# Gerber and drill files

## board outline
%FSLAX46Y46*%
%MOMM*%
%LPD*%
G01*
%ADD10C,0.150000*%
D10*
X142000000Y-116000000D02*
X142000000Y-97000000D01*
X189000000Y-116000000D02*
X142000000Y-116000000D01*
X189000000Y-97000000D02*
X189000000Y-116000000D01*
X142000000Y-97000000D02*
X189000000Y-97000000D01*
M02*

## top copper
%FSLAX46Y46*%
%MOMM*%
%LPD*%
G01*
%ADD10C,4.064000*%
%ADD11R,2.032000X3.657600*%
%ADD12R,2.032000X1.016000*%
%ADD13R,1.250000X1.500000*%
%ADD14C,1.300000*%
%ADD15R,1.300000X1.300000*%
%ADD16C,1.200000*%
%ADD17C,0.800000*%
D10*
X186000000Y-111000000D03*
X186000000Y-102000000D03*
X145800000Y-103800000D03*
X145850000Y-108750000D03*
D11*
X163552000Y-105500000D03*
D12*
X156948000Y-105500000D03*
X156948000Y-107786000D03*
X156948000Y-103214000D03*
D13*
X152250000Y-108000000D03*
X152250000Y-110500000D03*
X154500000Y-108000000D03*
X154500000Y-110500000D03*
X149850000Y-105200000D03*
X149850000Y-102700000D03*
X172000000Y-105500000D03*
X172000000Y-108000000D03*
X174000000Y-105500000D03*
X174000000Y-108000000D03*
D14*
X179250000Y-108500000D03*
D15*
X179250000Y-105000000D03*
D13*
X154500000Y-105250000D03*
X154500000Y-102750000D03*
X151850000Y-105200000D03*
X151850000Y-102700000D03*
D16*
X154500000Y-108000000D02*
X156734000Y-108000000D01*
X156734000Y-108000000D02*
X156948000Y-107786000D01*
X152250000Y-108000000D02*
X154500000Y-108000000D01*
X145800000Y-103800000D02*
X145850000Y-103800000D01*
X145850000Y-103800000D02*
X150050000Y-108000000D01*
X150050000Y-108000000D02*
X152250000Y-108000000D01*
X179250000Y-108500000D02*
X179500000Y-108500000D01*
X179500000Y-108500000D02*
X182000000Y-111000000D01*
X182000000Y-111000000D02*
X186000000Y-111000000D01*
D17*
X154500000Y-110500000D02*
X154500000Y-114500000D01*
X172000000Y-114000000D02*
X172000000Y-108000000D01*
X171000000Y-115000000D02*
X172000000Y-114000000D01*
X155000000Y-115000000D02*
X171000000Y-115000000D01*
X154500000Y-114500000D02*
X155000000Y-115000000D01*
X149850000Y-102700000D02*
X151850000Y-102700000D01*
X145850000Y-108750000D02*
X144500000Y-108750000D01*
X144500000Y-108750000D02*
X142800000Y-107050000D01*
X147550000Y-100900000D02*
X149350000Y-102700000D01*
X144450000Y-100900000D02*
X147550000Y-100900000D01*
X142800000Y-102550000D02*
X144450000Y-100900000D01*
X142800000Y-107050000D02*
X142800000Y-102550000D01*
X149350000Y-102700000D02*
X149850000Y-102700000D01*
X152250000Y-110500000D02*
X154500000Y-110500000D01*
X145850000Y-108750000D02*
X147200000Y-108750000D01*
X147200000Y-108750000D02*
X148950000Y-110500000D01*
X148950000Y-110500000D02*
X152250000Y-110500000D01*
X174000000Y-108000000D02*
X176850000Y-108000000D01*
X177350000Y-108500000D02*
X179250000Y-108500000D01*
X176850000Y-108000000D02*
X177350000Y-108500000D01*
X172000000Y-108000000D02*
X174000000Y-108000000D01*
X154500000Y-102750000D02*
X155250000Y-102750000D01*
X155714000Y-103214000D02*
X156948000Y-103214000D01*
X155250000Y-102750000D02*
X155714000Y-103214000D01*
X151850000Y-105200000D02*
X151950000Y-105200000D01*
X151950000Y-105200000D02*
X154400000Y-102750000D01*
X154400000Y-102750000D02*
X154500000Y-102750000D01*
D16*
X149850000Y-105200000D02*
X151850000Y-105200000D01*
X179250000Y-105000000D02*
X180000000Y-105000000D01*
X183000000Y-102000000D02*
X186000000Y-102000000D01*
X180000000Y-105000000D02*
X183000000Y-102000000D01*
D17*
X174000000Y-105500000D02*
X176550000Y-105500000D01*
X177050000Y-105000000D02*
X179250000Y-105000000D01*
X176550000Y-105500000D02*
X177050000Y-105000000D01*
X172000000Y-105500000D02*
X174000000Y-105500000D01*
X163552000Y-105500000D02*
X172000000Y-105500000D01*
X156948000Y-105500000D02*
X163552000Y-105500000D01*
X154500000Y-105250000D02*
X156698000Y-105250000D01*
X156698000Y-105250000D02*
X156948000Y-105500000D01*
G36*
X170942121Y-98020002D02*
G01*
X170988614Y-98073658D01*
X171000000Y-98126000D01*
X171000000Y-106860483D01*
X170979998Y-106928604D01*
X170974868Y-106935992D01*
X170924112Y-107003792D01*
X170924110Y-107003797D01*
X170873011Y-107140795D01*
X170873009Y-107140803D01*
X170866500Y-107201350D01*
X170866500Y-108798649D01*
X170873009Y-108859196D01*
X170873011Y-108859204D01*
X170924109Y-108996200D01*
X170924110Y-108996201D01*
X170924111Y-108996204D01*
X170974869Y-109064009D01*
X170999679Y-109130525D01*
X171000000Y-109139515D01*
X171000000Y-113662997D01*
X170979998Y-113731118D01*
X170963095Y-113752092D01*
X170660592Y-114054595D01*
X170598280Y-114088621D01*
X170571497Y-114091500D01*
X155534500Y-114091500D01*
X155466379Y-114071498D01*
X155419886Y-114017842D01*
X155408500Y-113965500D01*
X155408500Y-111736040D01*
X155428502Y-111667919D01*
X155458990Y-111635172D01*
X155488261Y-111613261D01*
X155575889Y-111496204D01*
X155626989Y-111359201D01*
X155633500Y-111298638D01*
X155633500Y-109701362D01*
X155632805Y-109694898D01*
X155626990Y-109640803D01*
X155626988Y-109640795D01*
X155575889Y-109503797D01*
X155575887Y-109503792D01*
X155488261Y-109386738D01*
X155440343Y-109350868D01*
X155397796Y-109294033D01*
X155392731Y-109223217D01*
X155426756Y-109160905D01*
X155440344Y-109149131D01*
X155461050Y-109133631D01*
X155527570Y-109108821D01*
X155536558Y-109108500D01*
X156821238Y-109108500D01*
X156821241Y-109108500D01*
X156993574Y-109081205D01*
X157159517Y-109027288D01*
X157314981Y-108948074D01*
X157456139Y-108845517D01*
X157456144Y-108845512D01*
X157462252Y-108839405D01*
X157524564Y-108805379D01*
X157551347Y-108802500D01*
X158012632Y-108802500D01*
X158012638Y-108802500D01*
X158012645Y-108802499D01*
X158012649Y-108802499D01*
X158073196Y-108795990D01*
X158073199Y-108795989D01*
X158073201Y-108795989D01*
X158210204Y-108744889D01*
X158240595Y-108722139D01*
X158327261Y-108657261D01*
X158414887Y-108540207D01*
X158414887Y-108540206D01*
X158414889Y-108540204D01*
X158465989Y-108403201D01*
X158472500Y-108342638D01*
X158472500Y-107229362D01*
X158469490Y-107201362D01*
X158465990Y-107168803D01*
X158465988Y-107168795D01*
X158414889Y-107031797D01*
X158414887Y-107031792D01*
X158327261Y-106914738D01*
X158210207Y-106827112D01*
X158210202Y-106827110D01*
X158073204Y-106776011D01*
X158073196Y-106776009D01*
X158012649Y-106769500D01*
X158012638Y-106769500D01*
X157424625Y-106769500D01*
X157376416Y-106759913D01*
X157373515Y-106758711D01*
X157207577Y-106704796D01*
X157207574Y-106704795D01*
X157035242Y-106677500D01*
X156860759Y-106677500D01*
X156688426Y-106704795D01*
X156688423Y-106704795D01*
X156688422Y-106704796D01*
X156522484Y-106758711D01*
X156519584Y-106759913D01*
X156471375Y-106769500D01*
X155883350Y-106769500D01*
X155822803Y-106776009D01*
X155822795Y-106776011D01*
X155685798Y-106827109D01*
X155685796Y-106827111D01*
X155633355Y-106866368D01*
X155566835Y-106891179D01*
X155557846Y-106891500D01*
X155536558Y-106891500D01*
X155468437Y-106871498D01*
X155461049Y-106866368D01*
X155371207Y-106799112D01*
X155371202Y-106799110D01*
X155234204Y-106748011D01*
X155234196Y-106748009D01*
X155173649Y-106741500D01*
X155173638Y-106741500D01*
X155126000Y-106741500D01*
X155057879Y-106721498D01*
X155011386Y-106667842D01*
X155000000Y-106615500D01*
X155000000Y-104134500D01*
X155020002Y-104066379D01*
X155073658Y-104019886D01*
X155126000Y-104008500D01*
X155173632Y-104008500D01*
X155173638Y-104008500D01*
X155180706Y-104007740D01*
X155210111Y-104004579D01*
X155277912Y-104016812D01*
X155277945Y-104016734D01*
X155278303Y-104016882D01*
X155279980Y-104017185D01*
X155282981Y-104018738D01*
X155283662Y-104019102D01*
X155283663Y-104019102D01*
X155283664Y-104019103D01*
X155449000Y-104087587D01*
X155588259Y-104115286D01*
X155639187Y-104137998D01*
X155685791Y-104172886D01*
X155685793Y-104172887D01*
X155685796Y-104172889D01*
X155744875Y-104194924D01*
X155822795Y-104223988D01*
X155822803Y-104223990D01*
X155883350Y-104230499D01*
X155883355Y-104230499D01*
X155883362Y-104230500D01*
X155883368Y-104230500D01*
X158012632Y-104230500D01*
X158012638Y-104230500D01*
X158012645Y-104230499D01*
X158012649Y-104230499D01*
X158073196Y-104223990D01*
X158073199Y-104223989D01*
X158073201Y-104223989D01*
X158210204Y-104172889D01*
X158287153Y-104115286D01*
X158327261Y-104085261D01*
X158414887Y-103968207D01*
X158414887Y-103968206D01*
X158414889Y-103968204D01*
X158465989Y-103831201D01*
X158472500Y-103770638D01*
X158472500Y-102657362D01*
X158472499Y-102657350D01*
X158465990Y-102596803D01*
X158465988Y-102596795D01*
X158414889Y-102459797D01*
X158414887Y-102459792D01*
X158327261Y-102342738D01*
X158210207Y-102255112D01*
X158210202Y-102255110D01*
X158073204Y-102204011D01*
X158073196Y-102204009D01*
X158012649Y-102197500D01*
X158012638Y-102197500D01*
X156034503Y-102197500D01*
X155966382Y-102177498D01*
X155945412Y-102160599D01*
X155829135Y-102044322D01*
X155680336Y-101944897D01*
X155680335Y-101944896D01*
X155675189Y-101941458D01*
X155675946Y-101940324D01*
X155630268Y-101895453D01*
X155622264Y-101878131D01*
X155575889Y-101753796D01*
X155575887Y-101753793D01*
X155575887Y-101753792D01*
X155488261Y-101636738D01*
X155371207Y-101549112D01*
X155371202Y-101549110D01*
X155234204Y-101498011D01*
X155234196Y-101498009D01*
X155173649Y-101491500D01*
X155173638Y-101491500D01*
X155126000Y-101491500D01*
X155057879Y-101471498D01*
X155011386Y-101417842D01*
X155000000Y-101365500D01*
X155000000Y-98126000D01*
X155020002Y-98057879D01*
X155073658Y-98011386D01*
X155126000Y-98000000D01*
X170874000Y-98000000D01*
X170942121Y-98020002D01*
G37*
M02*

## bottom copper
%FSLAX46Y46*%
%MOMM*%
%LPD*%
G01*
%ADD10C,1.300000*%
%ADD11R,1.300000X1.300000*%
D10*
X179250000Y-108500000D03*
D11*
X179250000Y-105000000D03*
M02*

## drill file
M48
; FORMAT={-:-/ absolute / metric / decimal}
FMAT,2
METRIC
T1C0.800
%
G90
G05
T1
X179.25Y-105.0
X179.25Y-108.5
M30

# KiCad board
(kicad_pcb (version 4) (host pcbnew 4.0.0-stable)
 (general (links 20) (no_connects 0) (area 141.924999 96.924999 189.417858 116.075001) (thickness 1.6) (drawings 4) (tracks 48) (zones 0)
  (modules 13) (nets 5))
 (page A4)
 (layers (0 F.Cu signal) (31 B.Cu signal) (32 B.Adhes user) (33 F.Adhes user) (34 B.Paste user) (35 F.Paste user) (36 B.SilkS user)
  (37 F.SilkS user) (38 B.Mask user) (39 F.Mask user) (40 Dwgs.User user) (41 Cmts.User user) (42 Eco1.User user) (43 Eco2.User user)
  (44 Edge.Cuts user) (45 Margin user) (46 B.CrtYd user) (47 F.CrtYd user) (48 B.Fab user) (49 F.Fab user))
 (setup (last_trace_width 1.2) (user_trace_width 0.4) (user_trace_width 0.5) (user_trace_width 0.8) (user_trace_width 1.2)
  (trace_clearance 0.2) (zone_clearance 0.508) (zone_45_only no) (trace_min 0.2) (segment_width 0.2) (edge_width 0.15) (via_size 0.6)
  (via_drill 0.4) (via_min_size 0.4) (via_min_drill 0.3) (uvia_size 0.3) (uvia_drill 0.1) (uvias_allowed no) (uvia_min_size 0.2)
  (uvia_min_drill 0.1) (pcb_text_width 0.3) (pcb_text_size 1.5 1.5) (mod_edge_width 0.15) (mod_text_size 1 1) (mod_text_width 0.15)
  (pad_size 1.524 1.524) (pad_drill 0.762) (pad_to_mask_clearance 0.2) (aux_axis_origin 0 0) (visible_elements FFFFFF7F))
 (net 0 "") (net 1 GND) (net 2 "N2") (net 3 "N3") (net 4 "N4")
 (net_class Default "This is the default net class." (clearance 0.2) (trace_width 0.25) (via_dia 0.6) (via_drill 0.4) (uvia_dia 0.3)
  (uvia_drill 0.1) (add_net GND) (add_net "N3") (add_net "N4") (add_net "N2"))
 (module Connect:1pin (layer F.Cu) (at 186 111)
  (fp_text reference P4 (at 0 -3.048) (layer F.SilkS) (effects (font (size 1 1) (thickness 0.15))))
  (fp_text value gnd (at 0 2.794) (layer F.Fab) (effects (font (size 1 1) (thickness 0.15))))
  (pad 1 smd circle (at 0 0) (size 4.064 4.064) (layers F.Cu F.Paste F.Mask) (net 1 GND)))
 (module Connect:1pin (layer F.Cu) (at 186 102)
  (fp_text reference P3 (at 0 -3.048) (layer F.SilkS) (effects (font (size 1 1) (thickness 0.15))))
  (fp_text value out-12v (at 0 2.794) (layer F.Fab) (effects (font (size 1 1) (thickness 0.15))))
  (pad 1 smd circle (at 0 0) (size 4.064 4.064) (layers F.Cu F.Paste F.Mask) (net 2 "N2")))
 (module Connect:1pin (layer F.Cu) (at 145.8 103.8)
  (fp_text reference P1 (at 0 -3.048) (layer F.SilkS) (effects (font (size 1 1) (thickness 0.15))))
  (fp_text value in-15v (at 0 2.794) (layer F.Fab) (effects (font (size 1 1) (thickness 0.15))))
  (pad 1 smd circle (at 0 0) (size 4.064 4.064) (layers F.Cu F.Paste F.Mask) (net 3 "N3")))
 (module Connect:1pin (layer F.Cu) (at 145.85 108.75)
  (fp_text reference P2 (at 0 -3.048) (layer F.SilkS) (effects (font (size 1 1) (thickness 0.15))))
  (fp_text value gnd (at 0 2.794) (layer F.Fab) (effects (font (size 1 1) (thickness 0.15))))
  (pad 1 smd circle (at 0 0) (size 4.064 4.064) (layers F.Cu F.Paste F.Mask) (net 1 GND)))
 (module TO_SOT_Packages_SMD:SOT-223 (layer F.Cu) (at 160.25 105.5 270)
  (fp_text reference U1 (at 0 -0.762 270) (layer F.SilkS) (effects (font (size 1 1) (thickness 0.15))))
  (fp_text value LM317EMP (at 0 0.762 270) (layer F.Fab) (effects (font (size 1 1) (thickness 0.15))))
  (pad 2 smd rect (at 0 -3.302 270) (size 3.6576 2.032) (layers F.Cu F.Paste F.Mask) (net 2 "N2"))
  (pad 2 smd rect (at 0 3.302 270) (size 1.016 2.032) (layers F.Cu F.Paste F.Mask) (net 2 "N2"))
  (pad 3 smd rect (at 2.286 3.302 270) (size 1.016 2.032) (layers F.Cu F.Paste F.Mask) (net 3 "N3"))
  (pad 1 smd rect (at -2.286 3.302 270) (size 1.016 2.032) (layers F.Cu F.Paste F.Mask) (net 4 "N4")))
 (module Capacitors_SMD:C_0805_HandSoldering (layer F.Cu) (at 152.25 109.25 270)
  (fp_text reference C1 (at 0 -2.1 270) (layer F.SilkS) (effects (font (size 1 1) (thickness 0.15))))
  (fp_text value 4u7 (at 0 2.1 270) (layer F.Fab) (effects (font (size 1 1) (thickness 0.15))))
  (pad 1 smd rect (at -1.25 0 270) (size 1.5 1.25) (layers F.Cu F.Paste F.Mask) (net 3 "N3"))
  (pad 2 smd rect (at 1.25 0 270) (size 1.5 1.25) (layers F.Cu F.Paste F.Mask) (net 1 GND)))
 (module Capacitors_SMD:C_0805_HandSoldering (layer F.Cu) (at 154.5 109.25 270)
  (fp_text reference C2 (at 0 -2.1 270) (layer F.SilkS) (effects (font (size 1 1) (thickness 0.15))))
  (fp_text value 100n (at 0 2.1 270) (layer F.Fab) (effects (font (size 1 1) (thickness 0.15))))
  (pad 1 smd rect (at -1.25 0 270) (size 1.5 1.25) (layers F.Cu F.Paste F.Mask) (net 3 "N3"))
  (pad 2 smd rect (at 1.25 0 270) (size 1.5 1.25) (layers F.Cu F.Paste F.Mask) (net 1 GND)))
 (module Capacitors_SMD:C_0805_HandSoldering (layer F.Cu) (at 149.85 103.95 90)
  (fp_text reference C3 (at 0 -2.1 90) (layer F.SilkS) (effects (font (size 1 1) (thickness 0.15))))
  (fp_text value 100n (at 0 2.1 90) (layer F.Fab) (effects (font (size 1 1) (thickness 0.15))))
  (pad 1 smd rect (at -1.25 0 90) (size 1.5 1.25) (layers F.Cu F.Paste F.Mask) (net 4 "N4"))
  (pad 2 smd rect (at 1.25 0 90) (size 1.5 1.25) (layers F.Cu F.Paste F.Mask) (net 1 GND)))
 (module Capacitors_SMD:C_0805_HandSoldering (layer F.Cu) (at 172 106.75 270)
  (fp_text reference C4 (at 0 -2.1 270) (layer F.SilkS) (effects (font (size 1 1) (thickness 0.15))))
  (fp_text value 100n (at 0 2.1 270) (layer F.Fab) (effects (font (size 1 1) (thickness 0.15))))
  (pad 1 smd rect (at -1.25 0 270) (size 1.5 1.25) (layers F.Cu F.Paste F.Mask) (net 2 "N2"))
  (pad 2 smd rect (at 1.25 0 270) (size 1.5 1.25) (layers F.Cu F.Paste F.Mask) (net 1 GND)))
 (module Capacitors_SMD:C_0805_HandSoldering (layer F.Cu) (at 174 106.75 270)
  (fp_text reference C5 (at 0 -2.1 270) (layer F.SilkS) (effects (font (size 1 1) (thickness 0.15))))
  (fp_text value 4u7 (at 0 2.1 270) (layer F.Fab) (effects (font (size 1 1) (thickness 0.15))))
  (pad 1 smd rect (at -1.25 0 270) (size 1.5 1.25) (layers F.Cu F.Paste F.Mask) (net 2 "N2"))
  (pad 2 smd rect (at 1.25 0 270) (size 1.5 1.25) (layers F.Cu F.Paste F.Mask) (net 1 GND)))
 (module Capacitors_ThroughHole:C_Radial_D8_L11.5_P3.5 (layer F.Cu) (at 179.25 105 270)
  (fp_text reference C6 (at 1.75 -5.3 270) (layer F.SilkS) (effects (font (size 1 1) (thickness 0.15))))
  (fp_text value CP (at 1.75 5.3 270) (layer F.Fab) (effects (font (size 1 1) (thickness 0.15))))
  (pad 2 thru_hole circle (at 3.5 0 270) (size 1.3 1.3) (drill 0.8) (layers *.Cu *.Mask F.SilkS) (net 1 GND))
  (pad 1 thru_hole rect (at 0 0 270) (size 1.3 1.3) (drill 0.8) (layers *.Cu *.Mask F.SilkS) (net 2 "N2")))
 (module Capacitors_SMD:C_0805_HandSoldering (layer F.Cu) (at 154.5 104 90)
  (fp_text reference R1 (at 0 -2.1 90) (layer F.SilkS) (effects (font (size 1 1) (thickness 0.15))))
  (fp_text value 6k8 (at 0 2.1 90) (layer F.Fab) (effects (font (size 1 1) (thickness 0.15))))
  (pad 1 smd rect (at -1.25 0 90) (size 1.5 1.25) (layers F.Cu F.Paste F.Mask) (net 2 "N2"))
  (pad 2 smd rect (at 1.25 0 90) (size 1.5 1.25) (layers F.Cu F.Paste F.Mask) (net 4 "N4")))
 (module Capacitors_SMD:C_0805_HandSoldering (layer F.Cu) (at 151.85 103.95 90)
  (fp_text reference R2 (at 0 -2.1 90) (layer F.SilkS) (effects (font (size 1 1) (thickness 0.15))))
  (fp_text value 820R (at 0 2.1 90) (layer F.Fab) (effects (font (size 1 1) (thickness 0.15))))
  (pad 1 smd rect (at -1.25 0 90) (size 1.5 1.25) (layers F.Cu F.Paste F.Mask) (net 4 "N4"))
  (pad 2 smd rect (at 1.25 0 90) (size 1.5 1.25) (layers F.Cu F.Paste F.Mask) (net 1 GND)))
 (gr_line (start 142 116) (end 142 97) (angle 90) (layer Edge.Cuts) (width 0.15))
 (gr_line (start 189 116) (end 142 116) (angle 90) (layer Edge.Cuts) (width 0.15))
 (gr_line (start 189 97) (end 189 116) (angle 90) (layer Edge.Cuts) (width 0.15))
 (gr_line (start 142 97) (end 189 97) (angle 90) (layer Edge.Cuts) (width 0.15))
 (segment (start 154.5 108) (end 156.734 108) (width 1.2) (layer F.Cu) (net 3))
 (segment (start 156.734 108) (end 156.948 107.786) (width 1.2) (layer F.Cu) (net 3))
 (segment (start 152.25 108) (end 154.5 108) (width 1.2) (layer F.Cu) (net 3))
 (segment (start 145.8 103.8) (end 145.85 103.8) (width 1.2) (layer F.Cu) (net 3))
 (segment (start 145.85 103.8) (end 150.05 108) (width 1.2) (layer F.Cu) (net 3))
 (segment (start 150.05 108) (end 152.25 108) (width 1.2) (layer F.Cu) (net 3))
 (segment (start 179.25 108.5) (end 179.5 108.5) (width 1.2) (layer F.Cu) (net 1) (status C00000))
 (segment (start 179.5 108.5) (end 182 111) (width 1.2) (layer F.Cu) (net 1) (status 400000))
 (segment (start 182 111) (end 186 111) (width 1.2) (layer F.Cu) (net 1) (status 800000))
 (segment (start 154.5 110.5) (end 154.5 114.5) (width 0.8) (layer F.Cu) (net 1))
 (segment (start 172 114) (end 172 108) (width 0.8) (layer F.Cu) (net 1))
 (segment (start 171 115) (end 172 114) (width 0.8) (layer F.Cu) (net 1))
 (segment (start 155 115) (end 171 115) (width 0.8) (layer F.Cu) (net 1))
 (segment (start 154.5 114.5) (end 155 115) (width 0.8) (layer F.Cu) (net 1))
 (segment (start 149.85 102.7) (end 151.85 102.7) (width 0.8) (layer F.Cu) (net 1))
 (segment (start 145.85 108.75) (end 144.5 108.75) (width 0.8) (layer F.Cu) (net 1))
 (segment (start 144.5 108.75) (end 142.8 107.05) (width 0.8) (layer F.Cu) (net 1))
 (segment (start 147.55 100.9) (end 149.35 102.7) (width 0.8) (layer F.Cu) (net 1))
 (segment (start 144.45 100.9) (end 147.55 100.9) (width 0.8) (layer F.Cu) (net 1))
 (segment (start 142.8 102.55) (end 144.45 100.9) (width 0.8) (layer F.Cu) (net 1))
 (segment (start 142.8 107.05) (end 142.8 102.55) (width 0.8) (layer F.Cu) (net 1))
 (segment (start 149.35 102.7) (end 149.85 102.7) (width 0.8) (layer F.Cu) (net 1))
 (segment (start 152.25 110.5) (end 154.5 110.5) (width 0.8) (layer F.Cu) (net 1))
 (segment (start 145.85 108.75) (end 147.2 108.75) (width 0.8) (layer F.Cu) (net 1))
 (segment (start 147.2 108.75) (end 148.95 110.5) (width 0.8) (layer F.Cu) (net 1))
 (segment (start 148.95 110.5) (end 152.25 110.5) (width 0.8) (layer F.Cu) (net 1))
 (segment (start 174 108) (end 176.85 108) (width 0.8) (layer F.Cu) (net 1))
 (segment (start 177.35 108.5) (end 179.25 108.5) (width 0.8) (layer F.Cu) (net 1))
 (segment (start 176.85 108) (end 177.35 108.5) (width 0.8) (layer F.Cu) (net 1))
 (segment (start 172 108) (end 174 108) (width 0.8) (layer F.Cu) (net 1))
 (segment (start 154.5 102.75) (end 155.25 102.75) (width 0.8) (layer F.Cu) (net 4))
 (segment (start 155.714 103.214) (end 156.948 103.214) (width 0.8) (layer F.Cu) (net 4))
 (segment (start 155.25 102.75) (end 155.714 103.214) (width 0.8) (layer F.Cu) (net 4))
 (segment (start 151.85 105.2) (end 151.95 105.2) (width 0.8) (layer F.Cu) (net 4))
 (segment (start 151.95 105.2) (end 154.4 102.75) (width 0.8) (layer F.Cu) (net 4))
 (segment (start 154.4 102.75) (end 154.5 102.75) (width 0.8) (layer F.Cu) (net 4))
 (segment (start 149.85 105.2) (end 151.85 105.2) (width 1.2) (layer F.Cu) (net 4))
 (segment (start 179.25 105) (end 180 105) (width 1.2) (layer F.Cu) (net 2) (status 400000))
 (segment (start 183 102) (end 186 102) (width 1.2) (layer F.Cu) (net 2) (status 800000))
 (segment (start 180 105) (end 183 102) (width 1.2) (layer F.Cu) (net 2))
 (segment (start 174 105.5) (end 176.55 105.5) (width 0.8) (layer F.Cu) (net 2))
 (segment (start 177.05 105) (end 179.25 105) (width 0.8) (layer F.Cu) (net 2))
 (segment (start 176.55 105.5) (end 177.05 105) (width 0.8) (layer F.Cu) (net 2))
 (segment (start 172 105.5) (end 174 105.5) (width 0.8) (layer F.Cu) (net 2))
 (segment (start 163.552 105.5) (end 172 105.5) (width 0.8) (layer F.Cu) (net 2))
 (segment (start 156.948 105.5) (end 163.552 105.5) (width 0.8) (layer F.Cu) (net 2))
 (segment (start 154.5 105.25) (end 156.698 105.25) (width 0.8) (layer F.Cu) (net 2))
 (segment (start 156.698 105.25) (end 156.948 105.5) (width 0.8) (layer F.Cu) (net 2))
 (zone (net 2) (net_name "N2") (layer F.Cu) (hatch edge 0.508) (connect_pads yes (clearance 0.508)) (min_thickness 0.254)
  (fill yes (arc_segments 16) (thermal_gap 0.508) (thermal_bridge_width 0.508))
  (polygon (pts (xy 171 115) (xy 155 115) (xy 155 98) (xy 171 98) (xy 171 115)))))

